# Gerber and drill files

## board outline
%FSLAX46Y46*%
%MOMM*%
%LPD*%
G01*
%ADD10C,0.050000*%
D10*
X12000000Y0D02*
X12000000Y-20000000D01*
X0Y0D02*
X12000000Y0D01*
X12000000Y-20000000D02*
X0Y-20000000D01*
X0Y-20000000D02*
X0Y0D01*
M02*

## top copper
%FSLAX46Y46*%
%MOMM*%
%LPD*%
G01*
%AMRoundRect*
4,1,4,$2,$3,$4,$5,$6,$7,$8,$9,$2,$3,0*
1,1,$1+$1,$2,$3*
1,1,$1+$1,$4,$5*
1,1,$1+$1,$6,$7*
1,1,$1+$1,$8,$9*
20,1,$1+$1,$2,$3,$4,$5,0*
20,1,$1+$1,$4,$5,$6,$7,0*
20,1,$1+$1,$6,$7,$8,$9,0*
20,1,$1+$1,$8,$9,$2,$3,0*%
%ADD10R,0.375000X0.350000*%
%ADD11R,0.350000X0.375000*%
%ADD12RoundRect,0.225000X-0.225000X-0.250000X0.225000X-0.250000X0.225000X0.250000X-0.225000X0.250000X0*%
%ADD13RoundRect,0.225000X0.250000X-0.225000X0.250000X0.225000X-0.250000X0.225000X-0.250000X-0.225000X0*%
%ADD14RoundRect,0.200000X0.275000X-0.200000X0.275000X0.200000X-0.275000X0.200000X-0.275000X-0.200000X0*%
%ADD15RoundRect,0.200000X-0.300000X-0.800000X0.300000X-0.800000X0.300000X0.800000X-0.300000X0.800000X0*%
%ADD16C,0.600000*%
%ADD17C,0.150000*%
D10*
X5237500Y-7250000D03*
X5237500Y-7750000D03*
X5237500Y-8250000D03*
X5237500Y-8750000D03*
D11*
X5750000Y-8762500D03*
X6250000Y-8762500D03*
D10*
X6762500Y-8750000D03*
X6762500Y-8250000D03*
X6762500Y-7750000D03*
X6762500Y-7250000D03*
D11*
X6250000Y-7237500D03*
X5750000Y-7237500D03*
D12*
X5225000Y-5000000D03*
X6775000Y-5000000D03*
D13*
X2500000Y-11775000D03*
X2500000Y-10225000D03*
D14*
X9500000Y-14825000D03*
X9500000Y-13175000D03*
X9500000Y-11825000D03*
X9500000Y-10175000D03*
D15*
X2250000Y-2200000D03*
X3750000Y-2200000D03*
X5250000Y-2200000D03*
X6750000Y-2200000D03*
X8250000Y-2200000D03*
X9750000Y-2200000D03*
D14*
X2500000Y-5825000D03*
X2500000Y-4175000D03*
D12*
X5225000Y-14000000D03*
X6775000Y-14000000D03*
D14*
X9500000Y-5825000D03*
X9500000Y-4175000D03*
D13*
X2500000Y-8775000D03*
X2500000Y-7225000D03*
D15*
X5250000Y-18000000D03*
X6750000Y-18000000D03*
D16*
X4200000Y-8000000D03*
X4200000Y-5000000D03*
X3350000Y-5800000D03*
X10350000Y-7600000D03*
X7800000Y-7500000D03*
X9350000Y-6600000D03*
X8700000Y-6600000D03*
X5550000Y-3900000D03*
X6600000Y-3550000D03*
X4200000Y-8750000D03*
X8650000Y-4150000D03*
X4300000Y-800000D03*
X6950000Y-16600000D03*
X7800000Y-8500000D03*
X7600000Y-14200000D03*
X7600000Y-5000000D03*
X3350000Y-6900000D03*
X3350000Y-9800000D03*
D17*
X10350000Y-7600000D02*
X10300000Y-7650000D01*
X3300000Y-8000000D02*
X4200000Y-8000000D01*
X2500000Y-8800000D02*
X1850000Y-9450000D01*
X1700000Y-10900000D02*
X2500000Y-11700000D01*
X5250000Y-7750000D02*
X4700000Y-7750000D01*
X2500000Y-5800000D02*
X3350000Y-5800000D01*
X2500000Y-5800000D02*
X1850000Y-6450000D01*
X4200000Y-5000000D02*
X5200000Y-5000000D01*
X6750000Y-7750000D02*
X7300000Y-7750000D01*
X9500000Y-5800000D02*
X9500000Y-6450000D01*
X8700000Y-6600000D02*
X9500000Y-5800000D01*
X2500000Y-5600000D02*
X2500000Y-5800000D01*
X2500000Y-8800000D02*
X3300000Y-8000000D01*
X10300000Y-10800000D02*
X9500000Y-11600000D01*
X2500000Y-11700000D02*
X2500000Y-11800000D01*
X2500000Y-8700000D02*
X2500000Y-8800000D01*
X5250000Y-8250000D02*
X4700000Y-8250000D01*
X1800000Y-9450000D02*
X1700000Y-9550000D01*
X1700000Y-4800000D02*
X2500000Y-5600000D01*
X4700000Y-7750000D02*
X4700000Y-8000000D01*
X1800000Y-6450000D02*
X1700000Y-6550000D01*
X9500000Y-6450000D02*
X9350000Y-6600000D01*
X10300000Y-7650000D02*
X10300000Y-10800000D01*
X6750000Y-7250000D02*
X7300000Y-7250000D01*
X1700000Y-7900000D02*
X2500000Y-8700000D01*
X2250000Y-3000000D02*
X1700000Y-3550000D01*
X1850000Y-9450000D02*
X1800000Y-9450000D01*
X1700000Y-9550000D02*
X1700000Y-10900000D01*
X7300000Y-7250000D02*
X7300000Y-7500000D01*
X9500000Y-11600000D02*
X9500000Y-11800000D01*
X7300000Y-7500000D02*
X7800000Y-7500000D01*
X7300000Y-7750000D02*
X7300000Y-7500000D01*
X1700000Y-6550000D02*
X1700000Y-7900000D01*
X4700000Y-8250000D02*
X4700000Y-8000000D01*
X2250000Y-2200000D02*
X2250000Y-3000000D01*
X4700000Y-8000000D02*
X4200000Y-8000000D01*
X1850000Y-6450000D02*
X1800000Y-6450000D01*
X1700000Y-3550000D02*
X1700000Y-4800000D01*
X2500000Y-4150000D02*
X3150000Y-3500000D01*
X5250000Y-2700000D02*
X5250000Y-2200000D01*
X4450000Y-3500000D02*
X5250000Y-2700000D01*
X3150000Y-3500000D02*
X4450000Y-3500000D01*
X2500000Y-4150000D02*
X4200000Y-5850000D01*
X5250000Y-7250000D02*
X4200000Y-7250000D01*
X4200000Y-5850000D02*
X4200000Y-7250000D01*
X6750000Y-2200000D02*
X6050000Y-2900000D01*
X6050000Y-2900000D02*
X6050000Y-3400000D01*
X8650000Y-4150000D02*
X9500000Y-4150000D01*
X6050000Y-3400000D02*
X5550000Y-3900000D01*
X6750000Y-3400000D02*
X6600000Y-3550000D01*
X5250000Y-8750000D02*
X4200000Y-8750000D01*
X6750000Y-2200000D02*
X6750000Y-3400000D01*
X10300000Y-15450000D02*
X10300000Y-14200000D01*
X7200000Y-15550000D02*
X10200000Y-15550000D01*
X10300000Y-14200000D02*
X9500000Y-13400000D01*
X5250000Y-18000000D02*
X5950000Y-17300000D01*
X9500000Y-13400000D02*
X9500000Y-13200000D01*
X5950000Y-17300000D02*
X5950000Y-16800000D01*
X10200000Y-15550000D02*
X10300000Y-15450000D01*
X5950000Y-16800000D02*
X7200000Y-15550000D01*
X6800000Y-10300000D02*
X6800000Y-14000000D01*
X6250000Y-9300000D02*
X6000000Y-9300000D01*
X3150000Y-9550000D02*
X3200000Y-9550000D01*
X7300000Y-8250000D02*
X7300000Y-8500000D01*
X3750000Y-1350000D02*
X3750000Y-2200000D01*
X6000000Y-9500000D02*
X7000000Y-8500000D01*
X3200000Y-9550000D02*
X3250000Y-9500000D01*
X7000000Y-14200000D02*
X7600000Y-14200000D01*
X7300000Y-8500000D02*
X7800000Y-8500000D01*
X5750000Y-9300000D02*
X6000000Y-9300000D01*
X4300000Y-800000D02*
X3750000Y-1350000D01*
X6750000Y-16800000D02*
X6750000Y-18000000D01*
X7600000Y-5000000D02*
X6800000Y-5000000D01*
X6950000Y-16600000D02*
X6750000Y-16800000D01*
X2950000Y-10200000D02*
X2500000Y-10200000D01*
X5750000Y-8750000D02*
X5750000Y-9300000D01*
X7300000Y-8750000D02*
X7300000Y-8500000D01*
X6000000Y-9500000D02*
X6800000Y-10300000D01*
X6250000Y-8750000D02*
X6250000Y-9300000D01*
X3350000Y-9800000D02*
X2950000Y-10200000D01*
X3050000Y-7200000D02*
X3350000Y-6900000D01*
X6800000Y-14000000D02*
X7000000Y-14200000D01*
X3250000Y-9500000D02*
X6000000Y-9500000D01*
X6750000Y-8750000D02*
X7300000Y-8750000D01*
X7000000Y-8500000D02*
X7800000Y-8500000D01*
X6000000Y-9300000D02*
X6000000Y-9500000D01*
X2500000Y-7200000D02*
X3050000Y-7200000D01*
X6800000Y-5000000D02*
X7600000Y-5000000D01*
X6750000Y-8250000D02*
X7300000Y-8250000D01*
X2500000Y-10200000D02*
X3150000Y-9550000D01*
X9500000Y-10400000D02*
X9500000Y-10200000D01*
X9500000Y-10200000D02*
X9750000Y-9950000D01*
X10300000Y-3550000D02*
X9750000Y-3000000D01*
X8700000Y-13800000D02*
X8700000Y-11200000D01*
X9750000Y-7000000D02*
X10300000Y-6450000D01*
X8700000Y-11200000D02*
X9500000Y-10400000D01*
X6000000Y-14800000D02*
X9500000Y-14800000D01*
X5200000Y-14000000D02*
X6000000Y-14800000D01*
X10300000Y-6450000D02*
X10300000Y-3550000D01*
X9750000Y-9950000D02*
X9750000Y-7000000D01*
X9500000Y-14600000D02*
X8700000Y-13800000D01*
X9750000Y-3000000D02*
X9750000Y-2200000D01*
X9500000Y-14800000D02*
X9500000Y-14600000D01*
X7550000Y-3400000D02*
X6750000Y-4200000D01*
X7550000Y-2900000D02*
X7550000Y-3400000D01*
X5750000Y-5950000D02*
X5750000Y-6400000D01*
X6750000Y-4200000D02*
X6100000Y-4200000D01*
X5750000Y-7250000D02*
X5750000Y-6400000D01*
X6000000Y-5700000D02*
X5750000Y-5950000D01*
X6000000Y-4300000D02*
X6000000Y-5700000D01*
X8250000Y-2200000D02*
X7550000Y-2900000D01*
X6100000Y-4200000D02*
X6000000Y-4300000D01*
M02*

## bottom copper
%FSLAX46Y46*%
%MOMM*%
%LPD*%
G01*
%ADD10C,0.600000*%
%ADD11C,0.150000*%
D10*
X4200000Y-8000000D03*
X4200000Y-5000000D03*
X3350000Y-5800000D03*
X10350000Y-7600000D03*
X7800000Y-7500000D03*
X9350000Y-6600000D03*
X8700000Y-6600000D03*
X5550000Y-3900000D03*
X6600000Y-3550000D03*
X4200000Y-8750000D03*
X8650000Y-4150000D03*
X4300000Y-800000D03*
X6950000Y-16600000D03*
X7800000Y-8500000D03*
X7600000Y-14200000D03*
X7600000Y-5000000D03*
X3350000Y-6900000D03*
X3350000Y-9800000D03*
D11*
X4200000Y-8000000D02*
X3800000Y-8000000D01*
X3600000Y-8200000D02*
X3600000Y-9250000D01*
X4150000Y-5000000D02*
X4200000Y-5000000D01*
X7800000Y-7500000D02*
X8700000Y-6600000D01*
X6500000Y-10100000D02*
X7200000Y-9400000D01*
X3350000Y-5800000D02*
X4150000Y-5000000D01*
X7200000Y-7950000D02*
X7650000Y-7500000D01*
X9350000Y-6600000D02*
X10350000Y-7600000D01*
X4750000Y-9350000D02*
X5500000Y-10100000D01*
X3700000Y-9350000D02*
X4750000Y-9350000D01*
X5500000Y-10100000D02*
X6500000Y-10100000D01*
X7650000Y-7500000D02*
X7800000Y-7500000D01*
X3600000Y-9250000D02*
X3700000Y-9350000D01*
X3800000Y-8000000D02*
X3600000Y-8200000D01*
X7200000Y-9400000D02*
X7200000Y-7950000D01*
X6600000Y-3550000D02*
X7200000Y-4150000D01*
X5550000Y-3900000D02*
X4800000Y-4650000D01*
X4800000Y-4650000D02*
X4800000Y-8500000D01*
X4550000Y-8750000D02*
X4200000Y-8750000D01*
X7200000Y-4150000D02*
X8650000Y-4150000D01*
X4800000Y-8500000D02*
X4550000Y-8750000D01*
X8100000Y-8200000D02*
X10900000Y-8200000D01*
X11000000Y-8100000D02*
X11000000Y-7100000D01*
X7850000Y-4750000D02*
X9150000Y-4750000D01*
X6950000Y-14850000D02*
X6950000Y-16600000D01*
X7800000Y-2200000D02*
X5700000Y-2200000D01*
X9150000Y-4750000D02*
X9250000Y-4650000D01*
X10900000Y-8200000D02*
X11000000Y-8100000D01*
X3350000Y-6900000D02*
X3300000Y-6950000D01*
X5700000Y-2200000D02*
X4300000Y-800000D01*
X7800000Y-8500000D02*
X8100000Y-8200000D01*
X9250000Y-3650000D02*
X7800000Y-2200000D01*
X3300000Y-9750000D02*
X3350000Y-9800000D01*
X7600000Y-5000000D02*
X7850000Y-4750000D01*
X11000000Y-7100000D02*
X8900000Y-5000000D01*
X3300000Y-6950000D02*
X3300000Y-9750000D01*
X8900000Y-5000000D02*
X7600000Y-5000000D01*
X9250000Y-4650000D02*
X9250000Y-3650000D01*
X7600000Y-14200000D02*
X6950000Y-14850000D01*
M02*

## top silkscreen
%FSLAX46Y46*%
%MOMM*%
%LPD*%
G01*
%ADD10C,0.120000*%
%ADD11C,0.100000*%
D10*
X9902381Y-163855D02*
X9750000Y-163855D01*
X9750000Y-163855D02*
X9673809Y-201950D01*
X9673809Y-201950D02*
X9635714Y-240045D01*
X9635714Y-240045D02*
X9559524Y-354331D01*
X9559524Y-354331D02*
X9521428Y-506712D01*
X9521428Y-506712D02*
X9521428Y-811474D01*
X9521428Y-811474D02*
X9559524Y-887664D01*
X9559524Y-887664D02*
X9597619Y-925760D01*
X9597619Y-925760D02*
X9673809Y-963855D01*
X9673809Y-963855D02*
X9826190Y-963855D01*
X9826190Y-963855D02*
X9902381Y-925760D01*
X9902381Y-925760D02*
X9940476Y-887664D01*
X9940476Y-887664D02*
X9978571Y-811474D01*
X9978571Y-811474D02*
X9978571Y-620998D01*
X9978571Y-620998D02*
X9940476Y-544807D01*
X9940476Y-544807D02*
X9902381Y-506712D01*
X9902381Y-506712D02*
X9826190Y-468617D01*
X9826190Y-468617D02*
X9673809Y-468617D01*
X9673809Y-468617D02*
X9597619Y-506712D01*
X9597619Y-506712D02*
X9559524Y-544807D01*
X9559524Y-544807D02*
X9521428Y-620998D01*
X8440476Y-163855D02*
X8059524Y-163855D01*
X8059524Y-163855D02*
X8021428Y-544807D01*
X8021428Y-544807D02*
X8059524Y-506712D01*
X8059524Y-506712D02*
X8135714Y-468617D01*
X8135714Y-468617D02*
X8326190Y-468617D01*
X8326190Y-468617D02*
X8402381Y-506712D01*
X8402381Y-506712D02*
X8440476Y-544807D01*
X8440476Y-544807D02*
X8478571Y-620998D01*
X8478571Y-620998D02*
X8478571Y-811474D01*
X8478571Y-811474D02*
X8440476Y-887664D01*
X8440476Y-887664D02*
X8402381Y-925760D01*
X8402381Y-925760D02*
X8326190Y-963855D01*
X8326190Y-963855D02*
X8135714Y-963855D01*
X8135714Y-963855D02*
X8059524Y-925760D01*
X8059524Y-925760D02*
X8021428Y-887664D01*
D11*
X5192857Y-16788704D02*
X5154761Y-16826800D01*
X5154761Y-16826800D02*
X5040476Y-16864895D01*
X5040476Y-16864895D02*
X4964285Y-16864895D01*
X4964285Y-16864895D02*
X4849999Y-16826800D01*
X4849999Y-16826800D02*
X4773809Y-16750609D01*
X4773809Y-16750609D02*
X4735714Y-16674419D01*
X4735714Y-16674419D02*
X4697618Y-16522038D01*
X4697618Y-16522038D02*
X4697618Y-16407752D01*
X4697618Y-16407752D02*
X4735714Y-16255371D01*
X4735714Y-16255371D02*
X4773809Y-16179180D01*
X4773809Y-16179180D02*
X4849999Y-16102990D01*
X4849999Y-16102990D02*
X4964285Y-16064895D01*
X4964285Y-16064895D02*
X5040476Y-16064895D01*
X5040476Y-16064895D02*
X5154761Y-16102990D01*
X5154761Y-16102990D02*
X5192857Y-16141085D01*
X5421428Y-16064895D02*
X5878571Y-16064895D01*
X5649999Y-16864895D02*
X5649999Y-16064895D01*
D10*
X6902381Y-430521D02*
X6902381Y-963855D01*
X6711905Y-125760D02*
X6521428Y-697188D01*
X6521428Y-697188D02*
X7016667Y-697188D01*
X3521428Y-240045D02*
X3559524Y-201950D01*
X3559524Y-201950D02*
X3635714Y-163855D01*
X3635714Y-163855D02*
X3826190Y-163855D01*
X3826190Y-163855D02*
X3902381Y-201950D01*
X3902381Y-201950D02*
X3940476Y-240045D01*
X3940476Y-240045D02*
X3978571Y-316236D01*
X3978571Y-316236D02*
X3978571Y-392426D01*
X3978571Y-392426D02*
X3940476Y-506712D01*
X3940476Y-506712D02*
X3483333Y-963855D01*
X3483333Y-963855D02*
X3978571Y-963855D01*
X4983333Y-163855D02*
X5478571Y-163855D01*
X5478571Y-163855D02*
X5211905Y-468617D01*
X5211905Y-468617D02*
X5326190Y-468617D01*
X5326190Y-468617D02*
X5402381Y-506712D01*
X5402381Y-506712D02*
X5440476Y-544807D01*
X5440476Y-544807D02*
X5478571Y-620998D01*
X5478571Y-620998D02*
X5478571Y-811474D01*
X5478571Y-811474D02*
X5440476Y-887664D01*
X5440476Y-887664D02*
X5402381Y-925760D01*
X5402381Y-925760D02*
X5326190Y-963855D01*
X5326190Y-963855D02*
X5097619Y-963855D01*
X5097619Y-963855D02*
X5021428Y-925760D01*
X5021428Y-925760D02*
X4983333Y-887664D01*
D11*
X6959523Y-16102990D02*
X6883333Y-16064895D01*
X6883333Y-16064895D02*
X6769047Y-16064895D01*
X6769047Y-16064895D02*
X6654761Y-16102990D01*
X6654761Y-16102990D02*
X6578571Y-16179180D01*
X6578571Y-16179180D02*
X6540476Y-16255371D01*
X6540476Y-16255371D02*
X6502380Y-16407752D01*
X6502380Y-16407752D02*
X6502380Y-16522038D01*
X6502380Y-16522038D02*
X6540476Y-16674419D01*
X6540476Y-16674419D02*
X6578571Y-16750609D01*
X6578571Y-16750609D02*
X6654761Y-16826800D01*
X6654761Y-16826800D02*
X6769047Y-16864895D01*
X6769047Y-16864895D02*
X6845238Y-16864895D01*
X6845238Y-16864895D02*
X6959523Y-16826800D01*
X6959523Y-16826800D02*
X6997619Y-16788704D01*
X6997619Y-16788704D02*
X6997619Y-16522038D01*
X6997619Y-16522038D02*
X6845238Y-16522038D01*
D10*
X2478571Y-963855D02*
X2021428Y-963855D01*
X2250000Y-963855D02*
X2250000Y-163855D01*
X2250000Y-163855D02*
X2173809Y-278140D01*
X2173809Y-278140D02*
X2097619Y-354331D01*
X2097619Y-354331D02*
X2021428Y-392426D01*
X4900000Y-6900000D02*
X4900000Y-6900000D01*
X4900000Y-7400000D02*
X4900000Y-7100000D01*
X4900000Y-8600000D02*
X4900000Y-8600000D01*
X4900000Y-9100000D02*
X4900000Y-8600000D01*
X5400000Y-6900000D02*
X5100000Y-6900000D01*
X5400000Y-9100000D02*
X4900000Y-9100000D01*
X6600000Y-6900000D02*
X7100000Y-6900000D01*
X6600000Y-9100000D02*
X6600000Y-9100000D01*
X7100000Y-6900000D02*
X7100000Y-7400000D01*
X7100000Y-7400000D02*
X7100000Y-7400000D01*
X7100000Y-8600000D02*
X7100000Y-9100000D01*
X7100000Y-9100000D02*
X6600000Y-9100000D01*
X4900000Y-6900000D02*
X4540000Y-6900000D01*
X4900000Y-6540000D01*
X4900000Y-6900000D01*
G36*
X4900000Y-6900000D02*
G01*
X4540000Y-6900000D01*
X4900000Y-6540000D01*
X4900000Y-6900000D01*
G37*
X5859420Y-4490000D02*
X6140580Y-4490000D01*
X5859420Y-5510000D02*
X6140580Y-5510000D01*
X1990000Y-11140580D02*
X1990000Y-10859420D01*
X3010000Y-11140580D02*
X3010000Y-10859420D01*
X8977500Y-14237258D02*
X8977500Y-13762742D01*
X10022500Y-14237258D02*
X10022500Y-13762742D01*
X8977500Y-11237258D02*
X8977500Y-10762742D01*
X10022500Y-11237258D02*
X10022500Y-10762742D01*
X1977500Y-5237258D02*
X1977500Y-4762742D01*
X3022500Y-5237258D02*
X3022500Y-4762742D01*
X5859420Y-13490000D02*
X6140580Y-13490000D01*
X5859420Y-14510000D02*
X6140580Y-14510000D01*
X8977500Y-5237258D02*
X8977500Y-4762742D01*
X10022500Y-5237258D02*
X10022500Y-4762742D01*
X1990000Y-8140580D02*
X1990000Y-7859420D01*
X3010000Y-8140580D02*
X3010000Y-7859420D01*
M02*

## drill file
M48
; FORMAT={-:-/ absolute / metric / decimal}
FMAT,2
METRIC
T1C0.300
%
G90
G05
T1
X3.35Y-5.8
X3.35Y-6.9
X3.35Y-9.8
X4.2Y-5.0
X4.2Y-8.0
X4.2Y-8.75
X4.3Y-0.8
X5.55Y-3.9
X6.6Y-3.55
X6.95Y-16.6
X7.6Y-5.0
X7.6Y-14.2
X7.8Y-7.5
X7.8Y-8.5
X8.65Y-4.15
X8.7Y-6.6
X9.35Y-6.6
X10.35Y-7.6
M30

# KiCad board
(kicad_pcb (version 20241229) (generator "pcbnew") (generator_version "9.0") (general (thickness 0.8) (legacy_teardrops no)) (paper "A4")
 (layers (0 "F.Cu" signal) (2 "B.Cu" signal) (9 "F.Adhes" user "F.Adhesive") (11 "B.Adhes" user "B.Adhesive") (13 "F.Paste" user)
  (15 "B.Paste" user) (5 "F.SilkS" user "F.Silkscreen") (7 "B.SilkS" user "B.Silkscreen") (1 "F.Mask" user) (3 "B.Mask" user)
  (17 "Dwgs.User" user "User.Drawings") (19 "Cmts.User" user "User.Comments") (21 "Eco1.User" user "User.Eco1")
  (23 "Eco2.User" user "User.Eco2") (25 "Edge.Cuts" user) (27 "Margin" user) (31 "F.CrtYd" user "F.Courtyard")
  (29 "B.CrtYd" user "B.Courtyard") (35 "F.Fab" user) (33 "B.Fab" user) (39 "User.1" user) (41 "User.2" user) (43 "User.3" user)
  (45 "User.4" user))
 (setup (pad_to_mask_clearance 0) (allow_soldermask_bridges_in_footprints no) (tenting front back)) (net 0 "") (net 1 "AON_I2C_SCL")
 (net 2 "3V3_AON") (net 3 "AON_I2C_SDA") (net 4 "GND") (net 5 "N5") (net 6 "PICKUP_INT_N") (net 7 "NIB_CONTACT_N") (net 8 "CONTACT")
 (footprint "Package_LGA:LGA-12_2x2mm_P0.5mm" (layer "F.Cu") (at 6 8)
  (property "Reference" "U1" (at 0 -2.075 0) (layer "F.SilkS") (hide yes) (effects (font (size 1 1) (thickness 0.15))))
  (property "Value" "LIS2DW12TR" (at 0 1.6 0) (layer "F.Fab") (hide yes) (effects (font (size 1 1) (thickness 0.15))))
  (fp_line (start -1.1 -1.1) (end -1.1 -1.1) (stroke (width 0.12) (type solid)) (layer "F.SilkS"))
  (fp_line (start -1.1 -0.6) (end -1.1 -0.9) (stroke (width 0.12) (type solid)) (layer "F.SilkS"))
  (fp_line (start -1.1 0.6) (end -1.1 0.6) (stroke (width 0.12) (type solid)) (layer "F.SilkS"))
  (fp_line (start -1.1 1.1) (end -1.1 0.6) (stroke (width 0.12) (type solid)) (layer "F.SilkS"))
  (fp_line (start -0.6 -1.1) (end -0.9 -1.1) (stroke (width 0.12) (type solid)) (layer "F.SilkS"))
  (fp_line (start -0.6 1.1) (end -1.1 1.1) (stroke (width 0.12) (type solid)) (layer "F.SilkS"))
  (fp_line (start 0.6 -1.1) (end 1.1 -1.1) (stroke (width 0.12) (type solid)) (layer "F.SilkS"))
  (fp_line (start 0.6 1.1) (end 0.6 1.1) (stroke (width 0.12) (type solid)) (layer "F.SilkS"))
  (fp_line (start 1.1 -1.1) (end 1.1 -0.6) (stroke (width 0.12) (type solid)) (layer "F.SilkS"))
  (fp_line (start 1.1 -0.6) (end 1.1 -0.6) (stroke (width 0.12) (type solid)) (layer "F.SilkS"))
  (fp_line (start 1.1 0.6) (end 1.1 1.1) (stroke (width 0.12) (type solid)) (layer "F.SilkS"))
  (fp_line (start 1.1 1.1) (end 0.6 1.1) (stroke (width 0.12) (type solid)) (layer "F.SilkS"))
  (fp_poly
   (pts (xy -1.1 -1.1) (xy -1.46 -1.1) (xy -1.1 -1.46) (xy -1.1 -1.1)) (stroke (width 0.12) (type solid)) (fill yes) (layer "F.SilkS"))
  (pad "1" smd rect (at -0.7625 -0.75) (size 0.375 0.35) (layers "F.Cu" "F.Mask" "F.Paste") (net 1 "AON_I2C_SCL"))
  (pad "2" smd rect (at -0.7625 -0.25) (size 0.375 0.35) (layers "F.Cu" "F.Mask" "F.Paste") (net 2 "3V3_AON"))
  (pad "3" smd rect (at -0.7625 0.25) (size 0.375 0.35) (layers "F.Cu" "F.Mask" "F.Paste") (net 2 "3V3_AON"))
  (pad "4" smd rect (at -0.7625 0.75) (size 0.375 0.35) (layers "F.Cu" "F.Mask" "F.Paste") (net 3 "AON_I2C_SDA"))
  (pad "5" smd rect (at -0.25 0.7625 90) (size 0.375 0.35) (layers "F.Cu" "F.Mask" "F.Paste") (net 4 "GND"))
  (pad "6" smd rect (at 0.25 0.7625 90) (size 0.375 0.35) (layers "F.Cu" "F.Mask" "F.Paste") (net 4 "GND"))
  (pad "7" smd rect (at 0.7625 0.75) (size 0.375 0.35) (layers "F.Cu" "F.Mask" "F.Paste") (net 4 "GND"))
  (pad "8" smd rect (at 0.7625 0.25) (size 0.375 0.35) (layers "F.Cu" "F.Mask" "F.Paste") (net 4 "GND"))
  (pad "9" smd rect (at 0.7625 -0.25) (size 0.375 0.35) (layers "F.Cu" "F.Mask" "F.Paste") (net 2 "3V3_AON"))
  (pad "10" smd rect (at 0.7625 -0.75) (size 0.375 0.35) (layers "F.Cu" "F.Mask" "F.Paste") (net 2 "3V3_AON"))
  (pad "11" smd rect (at 0.25 -0.7625 90) (size 0.375 0.35) (layers "F.Cu" "F.Mask" "F.Paste") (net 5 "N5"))
  (pad "12" smd rect (at -0.25 -0.7625 90) (size 0.375 0.35) (layers "F.Cu" "F.Mask" "F.Paste") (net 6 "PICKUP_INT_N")))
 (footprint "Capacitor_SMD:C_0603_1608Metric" (layer "F.Cu") (at 6 5)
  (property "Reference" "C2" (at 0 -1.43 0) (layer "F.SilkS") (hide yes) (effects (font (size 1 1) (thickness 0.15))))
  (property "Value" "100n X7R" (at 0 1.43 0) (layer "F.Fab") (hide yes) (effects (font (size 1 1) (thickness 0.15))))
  (fp_line (start -0.14058 -0.51) (end 0.14058 -0.51) (stroke (width 0.12) (type solid)) (layer "F.SilkS"))
  (fp_line (start -0.14058 0.51) (end 0.14058 0.51) (stroke (width 0.12) (type solid)) (layer "F.SilkS"))
  (pad "1" smd roundrect (at -0.775 0) (size 0.9 0.95) (layers "F.Cu" "F.Mask" "F.Paste") (roundrect_rratio 0.25) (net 2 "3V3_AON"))
  (pad "2" smd roundrect (at 0.775 0) (size 0.9 0.95) (layers "F.Cu" "F.Mask" "F.Paste") (roundrect_rratio 0.25) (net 4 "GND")))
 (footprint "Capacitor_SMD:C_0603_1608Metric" (layer "F.Cu") (at 2.5 11 90)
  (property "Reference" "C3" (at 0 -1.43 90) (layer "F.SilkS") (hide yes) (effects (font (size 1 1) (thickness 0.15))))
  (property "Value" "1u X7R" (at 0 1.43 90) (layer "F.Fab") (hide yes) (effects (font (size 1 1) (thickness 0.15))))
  (fp_line (start -0.14058 -0.51) (end 0.14058 -0.51) (stroke (width 0.12) (type solid)) (layer "F.SilkS"))
  (fp_line (start -0.14058 0.51) (end 0.14058 0.51) (stroke (width 0.12) (type solid)) (layer "F.SilkS"))
  (pad "1" smd roundrect (at -0.775 0 90) (size 0.9 0.95) (layers "F.Cu" "F.Mask" "F.Paste") (roundrect_rratio 0.25) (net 2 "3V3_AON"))
  (pad "2" smd roundrect (at 0.775 0 90) (size 0.9 0.95) (layers "F.Cu" "F.Mask" "F.Paste") (roundrect_rratio 0.25) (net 4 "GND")))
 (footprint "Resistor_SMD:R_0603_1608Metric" (layer "F.Cu") (at 9.5 14 90)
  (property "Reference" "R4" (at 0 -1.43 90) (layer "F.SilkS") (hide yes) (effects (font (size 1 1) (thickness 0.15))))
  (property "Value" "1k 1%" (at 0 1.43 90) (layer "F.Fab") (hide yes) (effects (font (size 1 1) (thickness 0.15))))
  (fp_line (start -0.237258 -0.5225) (end 0.237258 -0.5225) (stroke (width 0.12) (type solid)) (layer "F.SilkS"))
  (fp_line (start -0.237258 0.5225) (end 0.237258 0.5225) (stroke (width 0.12) (type solid)) (layer "F.SilkS"))
  (pad "1" smd roundrect (at -0.825 0 90) (size 0.8 0.95) (layers "F.Cu" "F.Mask" "F.Paste") (roundrect_rratio 0.25) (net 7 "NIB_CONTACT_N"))
  (pad "2" smd roundrect (at 0.825 0 90) (size 0.8 0.95) (layers "F.Cu" "F.Mask" "F.Paste") (roundrect_rratio 0.25) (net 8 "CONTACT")))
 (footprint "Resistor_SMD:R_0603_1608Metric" (layer "F.Cu") (at 9.5 11 90)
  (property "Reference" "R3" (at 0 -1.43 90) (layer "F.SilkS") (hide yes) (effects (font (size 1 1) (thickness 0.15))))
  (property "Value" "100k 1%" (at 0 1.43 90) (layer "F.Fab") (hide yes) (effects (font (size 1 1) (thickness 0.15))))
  (fp_line (start -0.237258 -0.5225) (end 0.237258 -0.5225) (stroke (width 0.12) (type solid)) (layer "F.SilkS"))
  (fp_line (start -0.237258 0.5225) (end 0.237258 0.5225) (stroke (width 0.12) (type solid)) (layer "F.SilkS"))
  (pad "1" smd roundrect (at -0.825 0 90) (size 0.8 0.95) (layers "F.Cu" "F.Mask" "F.Paste") (roundrect_rratio 0.25) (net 2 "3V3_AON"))
  (pad "2" smd roundrect (at 0.825 0 90) (size 0.8 0.95) (layers "F.Cu" "F.Mask" "F.Paste") (roundrect_rratio 0.25) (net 7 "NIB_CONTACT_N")))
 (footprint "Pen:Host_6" (layer "F.Cu") (at 2.25 2.2)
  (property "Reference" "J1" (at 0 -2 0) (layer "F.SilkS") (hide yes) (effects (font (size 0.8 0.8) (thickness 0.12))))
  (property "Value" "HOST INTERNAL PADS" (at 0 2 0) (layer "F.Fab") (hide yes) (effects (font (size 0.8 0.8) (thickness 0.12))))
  (pad "1" smd roundrect (at 0 0) (size 1 2) (layers "F.Cu" "F.Mask") (roundrect_rratio 0.2) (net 2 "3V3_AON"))
  (pad "2" smd roundrect (at 1.5 0) (size 1 2) (layers "F.Cu" "F.Mask") (roundrect_rratio 0.2) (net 4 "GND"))
  (pad "3" smd roundrect (at 3 0) (size 1 2) (layers "F.Cu" "F.Mask") (roundrect_rratio 0.2) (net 1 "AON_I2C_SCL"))
  (pad "4" smd roundrect (at 4.5 0) (size 1 2) (layers "F.Cu" "F.Mask") (roundrect_rratio 0.2) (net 3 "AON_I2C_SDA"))
  (pad "5" smd roundrect (at 6 0) (size 1 2) (layers "F.Cu" "F.Mask") (roundrect_rratio 0.2) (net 6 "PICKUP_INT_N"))
  (pad "6" smd roundrect (at 7.5 0) (size 1 2) (layers "F.Cu" "F.Mask") (roundrect_rratio 0.2) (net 7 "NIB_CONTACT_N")))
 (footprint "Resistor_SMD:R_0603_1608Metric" (layer "F.Cu") (at 2.5 5 90)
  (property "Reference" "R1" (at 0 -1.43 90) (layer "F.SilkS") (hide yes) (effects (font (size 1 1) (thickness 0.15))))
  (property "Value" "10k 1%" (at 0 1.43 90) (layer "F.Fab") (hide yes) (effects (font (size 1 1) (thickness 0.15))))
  (fp_line (start -0.237258 -0.5225) (end 0.237258 -0.5225) (stroke (width 0.12) (type solid)) (layer "F.SilkS"))
  (fp_line (start -0.237258 0.5225) (end 0.237258 0.5225) (stroke (width 0.12) (type solid)) (layer "F.SilkS"))
  (pad "1" smd roundrect (at -0.825 0 90) (size 0.8 0.95) (layers "F.Cu" "F.Mask" "F.Paste") (roundrect_rratio 0.25) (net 2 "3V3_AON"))
  (pad "2" smd roundrect (at 0.825 0 90) (size 0.8 0.95) (layers "F.Cu" "F.Mask" "F.Paste") (roundrect_rratio 0.25) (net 1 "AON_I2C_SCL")))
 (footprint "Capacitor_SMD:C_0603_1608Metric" (layer "F.Cu") (at 6 14)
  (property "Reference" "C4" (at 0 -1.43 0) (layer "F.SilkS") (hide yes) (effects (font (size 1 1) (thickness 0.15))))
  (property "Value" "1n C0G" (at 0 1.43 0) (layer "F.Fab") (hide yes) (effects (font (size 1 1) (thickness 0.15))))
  (fp_line (start -0.14058 -0.51) (end 0.14058 -0.51) (stroke (width 0.12) (type solid)) (layer "F.SilkS"))
  (fp_line (start -0.14058 0.51) (end 0.14058 0.51) (stroke (width 0.12) (type solid)) (layer "F.SilkS"))
  (pad "1" smd roundrect (at -0.775 0) (size 0.9 0.95) (layers "F.Cu" "F.Mask" "F.Paste") (roundrect_rratio 0.25) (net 7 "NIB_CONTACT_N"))
  (pad "2" smd roundrect (at 0.775 0) (size 0.9 0.95) (layers "F.Cu" "F.Mask" "F.Paste") (roundrect_rratio 0.25) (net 4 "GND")))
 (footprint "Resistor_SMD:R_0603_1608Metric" (layer "F.Cu") (at 9.5 5 90)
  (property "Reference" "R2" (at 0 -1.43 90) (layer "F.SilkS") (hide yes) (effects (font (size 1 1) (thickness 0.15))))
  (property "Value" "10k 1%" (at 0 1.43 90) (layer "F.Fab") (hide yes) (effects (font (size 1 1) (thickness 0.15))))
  (fp_line (start -0.237258 -0.5225) (end 0.237258 -0.5225) (stroke (width 0.12) (type solid)) (layer "F.SilkS"))
  (fp_line (start -0.237258 0.5225) (end 0.237258 0.5225) (stroke (width 0.12) (type solid)) (layer "F.SilkS"))
  (pad "1" smd roundrect (at -0.825 0 90) (size 0.8 0.95) (layers "F.Cu" "F.Mask" "F.Paste") (roundrect_rratio 0.25) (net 2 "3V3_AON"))
  (pad "2" smd roundrect (at 0.825 0 90) (size 0.8 0.95) (layers "F.Cu" "F.Mask" "F.Paste") (roundrect_rratio 0.25) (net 3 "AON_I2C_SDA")))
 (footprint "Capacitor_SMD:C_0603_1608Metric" (layer "F.Cu") (at 2.5 8 90)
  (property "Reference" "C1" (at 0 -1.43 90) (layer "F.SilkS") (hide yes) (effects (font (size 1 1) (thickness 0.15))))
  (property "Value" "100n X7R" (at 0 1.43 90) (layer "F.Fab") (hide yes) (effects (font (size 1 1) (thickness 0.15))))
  (fp_line (start -0.14058 -0.51) (end 0.14058 -0.51) (stroke (width 0.12) (type solid)) (layer "F.SilkS"))
  (fp_line (start -0.14058 0.51) (end 0.14058 0.51) (stroke (width 0.12) (type solid)) (layer "F.SilkS"))
  (pad "1" smd roundrect (at -0.775 0 90) (size 0.9 0.95) (layers "F.Cu" "F.Mask" "F.Paste") (roundrect_rratio 0.25) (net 2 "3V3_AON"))
  (pad "2" smd roundrect (at 0.775 0 90) (size 0.9 0.95) (layers "F.Cu" "F.Mask" "F.Paste") (roundrect_rratio 0.25) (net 4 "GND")))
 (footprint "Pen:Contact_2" (layer "F.Cu") (at 5.25 18)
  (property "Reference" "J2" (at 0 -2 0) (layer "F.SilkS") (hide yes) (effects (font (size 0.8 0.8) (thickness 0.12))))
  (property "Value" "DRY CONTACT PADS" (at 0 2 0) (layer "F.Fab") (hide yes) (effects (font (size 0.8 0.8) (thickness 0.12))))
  (pad "1" smd roundrect (at 0 0) (size 1 2) (layers "F.Cu" "F.Mask") (roundrect_rratio 0.2) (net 8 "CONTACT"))
  (pad "2" smd roundrect (at 1.5 0) (size 1 2) (layers "F.Cu" "F.Mask") (roundrect_rratio 0.2) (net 4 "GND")))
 (gr_line (start 12 0) (end 12 20) (stroke (width 0.05) (type default)) (layer "Edge.Cuts"))
 (gr_line (start 0 0) (end 12 0) (stroke (width 0.05) (type default)) (layer "Edge.Cuts"))
 (gr_line (start 12 20) (end 0 20) (stroke (width 0.05) (type default)) (layer "Edge.Cuts"))
 (gr_line (start 0 20) (end 0 0) (stroke (width 0.05) (type default)) (layer "Edge.Cuts"))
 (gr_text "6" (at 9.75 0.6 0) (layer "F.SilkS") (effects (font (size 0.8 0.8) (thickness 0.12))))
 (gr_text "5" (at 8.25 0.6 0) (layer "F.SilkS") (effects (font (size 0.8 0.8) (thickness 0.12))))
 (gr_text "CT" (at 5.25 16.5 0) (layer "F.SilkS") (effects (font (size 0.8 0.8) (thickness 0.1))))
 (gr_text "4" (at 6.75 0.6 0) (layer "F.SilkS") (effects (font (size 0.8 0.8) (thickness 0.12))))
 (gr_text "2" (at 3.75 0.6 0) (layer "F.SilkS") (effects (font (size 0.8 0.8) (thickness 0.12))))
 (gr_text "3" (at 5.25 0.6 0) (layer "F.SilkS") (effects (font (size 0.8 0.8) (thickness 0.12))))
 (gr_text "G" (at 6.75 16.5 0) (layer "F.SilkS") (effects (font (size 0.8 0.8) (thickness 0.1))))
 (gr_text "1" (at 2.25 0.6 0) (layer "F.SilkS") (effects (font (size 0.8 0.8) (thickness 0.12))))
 (segment (start 10.35 7.6) (end 10.3 7.65) (width 0.15) (layer "F.Cu") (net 2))
 (segment (start 3.3 8) (end 4.2 8) (width 0.15) (layer "F.Cu") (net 2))
 (segment (start 2.5 8.8) (end 1.85 9.45) (width 0.15) (layer "F.Cu") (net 2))
 (segment (start 1.7 10.9) (end 2.5 11.7) (width 0.15) (layer "F.Cu") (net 2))
 (segment (start 5.25 7.75) (end 4.7 7.75) (width 0.15) (layer "F.Cu") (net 2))
 (segment (start 2.5 5.8) (end 3.35 5.8) (width 0.15) (layer "F.Cu") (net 2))
 (segment (start 2.5 5.8) (end 1.85 6.45) (width 0.15) (layer "F.Cu") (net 2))
 (segment (start 4.2 5) (end 5.2 5) (width 0.15) (layer "F.Cu") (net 2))
 (segment (start 6.75 7.75) (end 7.3 7.75) (width 0.15) (layer "F.Cu") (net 2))
 (segment (start 9.5 5.8) (end 9.5 6.45) (width 0.15) (layer "F.Cu") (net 2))
 (segment (start 8.7 6.6) (end 9.5 5.8) (width 0.15) (layer "F.Cu") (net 2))
 (segment (start 2.5 5.6) (end 2.5 5.8) (width 0.15) (layer "F.Cu") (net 2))
 (segment (start 2.5 8.8) (end 3.3 8) (width 0.15) (layer "F.Cu") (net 2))
 (segment (start 10.3 10.8) (end 9.5 11.6) (width 0.15) (layer "F.Cu") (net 2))
 (segment (start 2.5 11.7) (end 2.5 11.8) (width 0.15) (layer "F.Cu") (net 2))
 (segment (start 2.5 8.7) (end 2.5 8.8) (width 0.15) (layer "F.Cu") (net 2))
 (segment (start 5.25 8.25) (end 4.7 8.25) (width 0.15) (layer "F.Cu") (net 2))
 (segment (start 1.8 9.45) (end 1.7 9.55) (width 0.15) (layer "F.Cu") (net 2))
 (segment (start 1.7 4.8) (end 2.5 5.6) (width 0.15) (layer "F.Cu") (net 2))
 (segment (start 4.7 7.75) (end 4.7 8) (width 0.15) (layer "F.Cu") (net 2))
 (segment (start 1.8 6.45) (end 1.7 6.55) (width 0.15) (layer "F.Cu") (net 2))
 (segment (start 9.5 6.45) (end 9.35 6.6) (width 0.15) (layer "F.Cu") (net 2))
 (segment (start 10.3 7.65) (end 10.3 10.8) (width 0.15) (layer "F.Cu") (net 2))
 (segment (start 6.75 7.25) (end 7.3 7.25) (width 0.15) (layer "F.Cu") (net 2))
 (segment (start 1.7 7.9) (end 2.5 8.7) (width 0.15) (layer "F.Cu") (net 2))
 (segment (start 2.25 3) (end 1.7 3.55) (width 0.15) (layer "F.Cu") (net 2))
 (segment (start 1.85 9.45) (end 1.8 9.45) (width 0.15) (layer "F.Cu") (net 2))
 (segment (start 1.7 9.55) (end 1.7 10.9) (width 0.15) (layer "F.Cu") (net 2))
 (segment (start 7.3 7.25) (end 7.3 7.5) (width 0.15) (layer "F.Cu") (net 2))
 (segment (start 9.5 11.6) (end 9.5 11.8) (width 0.15) (layer "F.Cu") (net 2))
 (segment (start 7.3 7.5) (end 7.8 7.5) (width 0.15) (layer "F.Cu") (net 2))
 (segment (start 7.3 7.75) (end 7.3 7.5) (width 0.15) (layer "F.Cu") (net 2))
 (segment (start 1.7 6.55) (end 1.7 7.9) (width 0.15) (layer "F.Cu") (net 2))
 (segment (start 4.7 8.25) (end 4.7 8) (width 0.15) (layer "F.Cu") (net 2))
 (segment (start 2.25 2.2) (end 2.25 3) (width 0.15) (layer "F.Cu") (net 2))
 (segment (start 4.7 8) (end 4.2 8) (width 0.15) (layer "F.Cu") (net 2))
 (segment (start 1.85 6.45) (end 1.8 6.45) (width 0.15) (layer "F.Cu") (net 2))
 (segment (start 1.7 3.55) (end 1.7 4.8) (width 0.15) (layer "F.Cu") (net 2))
 (via (at 4.2 8) (size 0.6) (drill 0.3) (layers "F.Cu" "B.Cu") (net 2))
 (via (at 4.2 5) (size 0.6) (drill 0.3) (layers "F.Cu" "B.Cu") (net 2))
 (via (at 3.35 5.8) (size 0.6) (drill 0.3) (layers "F.Cu" "B.Cu") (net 2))
 (via (at 10.35 7.6) (size 0.6) (drill 0.3) (layers "F.Cu" "B.Cu") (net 2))
 (via (at 7.8 7.5) (size 0.6) (drill 0.3) (layers "F.Cu" "B.Cu") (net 2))
 (via (at 9.35 6.6) (size 0.6) (drill 0.3) (layers "F.Cu" "B.Cu") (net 2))
 (via (at 8.7 6.6) (size 0.6) (drill 0.3) (layers "F.Cu" "B.Cu") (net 2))
 (segment (start 4.2 8) (end 3.8 8) (width 0.15) (layer "B.Cu") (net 2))
 (segment (start 3.6 8.2) (end 3.6 9.25) (width 0.15) (layer "B.Cu") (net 2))
 (segment (start 4.15 5) (end 4.2 5) (width 0.15) (layer "B.Cu") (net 2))
 (segment (start 7.8 7.5) (end 8.7 6.6) (width 0.15) (layer "B.Cu") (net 2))
 (segment (start 6.5 10.1) (end 7.2 9.4) (width 0.15) (layer "B.Cu") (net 2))
 (segment (start 3.35 5.8) (end 4.15 5) (width 0.15) (layer "B.Cu") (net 2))
 (segment (start 7.2 7.95) (end 7.65 7.5) (width 0.15) (layer "B.Cu") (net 2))
 (segment (start 9.35 6.6) (end 10.35 7.6) (width 0.15) (layer "B.Cu") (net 2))
 (segment (start 4.75 9.35) (end 5.5 10.1) (width 0.15) (layer "B.Cu") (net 2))
 (segment (start 3.7 9.35) (end 4.75 9.35) (width 0.15) (layer "B.Cu") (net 2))
 (segment (start 5.5 10.1) (end 6.5 10.1) (width 0.15) (layer "B.Cu") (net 2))
 (segment (start 7.65 7.5) (end 7.8 7.5) (width 0.15) (layer "B.Cu") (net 2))
 (segment (start 3.6 9.25) (end 3.7 9.35) (width 0.15) (layer "B.Cu") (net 2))
 (segment (start 3.8 8) (end 3.6 8.2) (width 0.15) (layer "B.Cu") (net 2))
 (segment (start 7.2 9.4) (end 7.2 7.95) (width 0.15) (layer "B.Cu") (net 2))
 (segment (start 2.5 4.15) (end 3.15 3.5) (width 0.15) (layer "F.Cu") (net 1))
 (segment (start 5.25 2.7) (end 5.25 2.2) (width 0.15) (layer "F.Cu") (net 1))
 (segment (start 4.45 3.5) (end 5.25 2.7) (width 0.15) (layer "F.Cu") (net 1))
 (segment (start 3.15 3.5) (end 4.45 3.5) (width 0.15) (layer "F.Cu") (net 1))
 (segment (start 2.5 4.15) (end 4.2 5.85) (width 0.15) (layer "F.Cu") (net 1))
 (segment (start 5.25 7.25) (end 4.2 7.25) (width 0.15) (layer "F.Cu") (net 1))
 (segment (start 4.2 5.85) (end 4.2 7.25) (width 0.15) (layer "F.Cu") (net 1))
 (segment (start 6.75 2.2) (end 6.05 2.9) (width 0.15) (layer "F.Cu") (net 3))
 (segment (start 6.05 2.9) (end 6.05 3.4) (width 0.15) (layer "F.Cu") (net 3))
 (segment (start 8.65 4.15) (end 9.5 4.15) (width 0.15) (layer "F.Cu") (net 3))
 (segment (start 6.05 3.4) (end 5.55 3.9) (width 0.15) (layer "F.Cu") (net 3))
 (segment (start 6.75 3.4) (end 6.6 3.55) (width 0.15) (layer "F.Cu") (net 3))
 (segment (start 5.25 8.75) (end 4.2 8.75) (width 0.15) (layer "F.Cu") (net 3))
 (segment (start 6.75 2.2) (end 6.75 3.4) (width 0.15) (layer "F.Cu") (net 3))
 (via (at 5.55 3.9) (size 0.6) (drill 0.3) (layers "F.Cu" "B.Cu") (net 3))
 (via (at 6.6 3.55) (size 0.6) (drill 0.3) (layers "F.Cu" "B.Cu") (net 3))
 (via (at 4.2 8.75) (size 0.6) (drill 0.3) (layers "F.Cu" "B.Cu") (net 3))
 (via (at 8.65 4.15) (size 0.6) (drill 0.3) (layers "F.Cu" "B.Cu") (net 3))
 (segment (start 6.6 3.55) (end 7.2 4.15) (width 0.15) (layer "B.Cu") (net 3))
 (segment (start 5.55 3.9) (end 4.8 4.65) (width 0.15) (layer "B.Cu") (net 3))
 (segment (start 4.8 4.65) (end 4.8 8.5) (width 0.15) (layer "B.Cu") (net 3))
 (segment (start 4.55 8.75) (end 4.2 8.75) (width 0.15) (layer "B.Cu") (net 3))
 (segment (start 7.2 4.15) (end 8.65 4.15) (width 0.15) (layer "B.Cu") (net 3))
 (segment (start 4.8 8.5) (end 4.55 8.75) (width 0.15) (layer "B.Cu") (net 3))
 (segment (start 10.3 15.45) (end 10.3 14.2) (width 0.15) (layer "F.Cu") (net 8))
 (segment (start 7.2 15.55) (end 10.2 15.55) (width 0.15) (layer "F.Cu") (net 8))
 (segment (start 10.3 14.2) (end 9.5 13.4) (width 0.15) (layer "F.Cu") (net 8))
 (segment (start 5.25 18) (end 5.95 17.3) (width 0.15) (layer "F.Cu") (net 8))
 (segment (start 9.5 13.4) (end 9.5 13.2) (width 0.15) (layer "F.Cu") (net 8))
 (segment (start 5.95 17.3) (end 5.95 16.8) (width 0.15) (layer "F.Cu") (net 8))
 (segment (start 10.2 15.55) (end 10.3 15.45) (width 0.15) (layer "F.Cu") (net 8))
 (segment (start 5.95 16.8) (end 7.2 15.55) (width 0.15) (layer "F.Cu") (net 8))
 (segment (start 6.8 10.3) (end 6.8 14) (width 0.15) (layer "F.Cu") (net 4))
 (segment (start 6.25 9.3) (end 6 9.3) (width 0.15) (layer "F.Cu") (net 4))
 (segment (start 3.15 9.55) (end 3.2 9.55) (width 0.15) (layer "F.Cu") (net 4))
 (segment (start 7.3 8.25) (end 7.3 8.5) (width 0.15) (layer "F.Cu") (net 4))
 (segment (start 3.75 1.35) (end 3.75 2.2) (width 0.15) (layer "F.Cu") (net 4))
 (segment (start 6 9.5) (end 7 8.5) (width 0.15) (layer "F.Cu") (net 4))
 (segment (start 3.2 9.55) (end 3.25 9.5) (width 0.15) (layer "F.Cu") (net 4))
 (segment (start 7 14.2) (end 7.6 14.2) (width 0.15) (layer "F.Cu") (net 4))
 (segment (start 7.3 8.5) (end 7.8 8.5) (width 0.15) (layer "F.Cu") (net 4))
 (segment (start 5.75 9.3) (end 6 9.3) (width 0.15) (layer "F.Cu") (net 4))
 (segment (start 4.3 0.8) (end 3.75 1.35) (width 0.15) (layer "F.Cu") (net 4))
 (segment (start 6.75 16.8) (end 6.75 18) (width 0.15) (layer "F.Cu") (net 4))
 (segment (start 7.6 5) (end 6.8 5) (width 0.15) (layer "F.Cu") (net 4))
 (segment (start 6.95 16.6) (end 6.75 16.8) (width 0.15) (layer "F.Cu") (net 4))
 (segment (start 2.95 10.2) (end 2.5 10.2) (width 0.15) (layer "F.Cu") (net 4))
 (segment (start 5.75 8.75) (end 5.75 9.3) (width 0.15) (layer "F.Cu") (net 4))
 (segment (start 7.3 8.75) (end 7.3 8.5) (width 0.15) (layer "F.Cu") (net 4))
 (segment (start 6 9.5) (end 6.8 10.3) (width 0.15) (layer "F.Cu") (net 4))
 (segment (start 6.25 8.75) (end 6.25 9.3) (width 0.15) (layer "F.Cu") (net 4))
 (segment (start 3.35 9.8) (end 2.95 10.2) (width 0.15) (layer "F.Cu") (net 4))
 (segment (start 3.05 7.2) (end 3.35 6.9) (width 0.15) (layer "F.Cu") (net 4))
 (segment (start 6.8 14) (end 7 14.2) (width 0.15) (layer "F.Cu") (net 4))
 (segment (start 3.25 9.5) (end 6 9.5) (width 0.15) (layer "F.Cu") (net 4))
 (segment (start 6.75 8.75) (end 7.3 8.75) (width 0.15) (layer "F.Cu") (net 4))
 (segment (start 7 8.5) (end 7.8 8.5) (width 0.15) (layer "F.Cu") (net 4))
 (segment (start 6 9.3) (end 6 9.5) (width 0.15) (layer "F.Cu") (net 4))
 (segment (start 2.5 7.2) (end 3.05 7.2) (width 0.15) (layer "F.Cu") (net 4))
 (segment (start 6.8 5) (end 7.6 5) (width 0.15) (layer "F.Cu") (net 4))
 (segment (start 6.75 8.25) (end 7.3 8.25) (width 0.15) (layer "F.Cu") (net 4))
 (segment (start 2.5 10.2) (end 3.15 9.55) (width 0.15) (layer "F.Cu") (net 4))
 (via (at 4.3 0.8) (size 0.6) (drill 0.3) (layers "F.Cu" "B.Cu") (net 4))
 (via (at 6.95 16.6) (size 0.6) (drill 0.3) (layers "F.Cu" "B.Cu") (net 4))
 (via (at 7.8 8.5) (size 0.6) (drill 0.3) (layers "F.Cu" "B.Cu") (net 4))
 (via (at 7.6 14.2) (size 0.6) (drill 0.3) (layers "F.Cu" "B.Cu") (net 4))
 (via (at 7.6 5) (size 0.6) (drill 0.3) (layers "F.Cu" "B.Cu") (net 4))
 (via (at 3.35 6.9) (size 0.6) (drill 0.3) (layers "F.Cu" "B.Cu") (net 4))
 (via (at 3.35 9.8) (size 0.6) (drill 0.3) (layers "F.Cu" "B.Cu") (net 4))
 (segment (start 8.1 8.2) (end 10.9 8.2) (width 0.15) (layer "B.Cu") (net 4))
 (segment (start 11 8.1) (end 11 7.1) (width 0.15) (layer "B.Cu") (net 4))
 (segment (start 7.85 4.75) (end 9.15 4.75) (width 0.15) (layer "B.Cu") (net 4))
 (segment (start 6.95 14.85) (end 6.95 16.6) (width 0.15) (layer "B.Cu") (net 4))
 (segment (start 7.8 2.2) (end 5.7 2.2) (width 0.15) (layer "B.Cu") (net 4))
 (segment (start 9.15 4.75) (end 9.25 4.65) (width 0.15) (layer "B.Cu") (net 4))
 (segment (start 10.9 8.2) (end 11 8.1) (width 0.15) (layer "B.Cu") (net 4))
 (segment (start 3.35 6.9) (end 3.3 6.95) (width 0.15) (layer "B.Cu") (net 4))
 (segment (start 5.7 2.2) (end 4.3 0.8) (width 0.15) (layer "B.Cu") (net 4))
 (segment (start 7.8 8.5) (end 8.1 8.2) (width 0.15) (layer "B.Cu") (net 4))
 (segment (start 9.25 3.65) (end 7.8 2.2) (width 0.15) (layer "B.Cu") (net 4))
 (segment (start 3.3 9.75) (end 3.35 9.8) (width 0.15) (layer "B.Cu") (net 4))
 (segment (start 7.6 5) (end 7.85 4.75) (width 0.15) (layer "B.Cu") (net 4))
 (segment (start 11 7.1) (end 8.9 5) (width 0.15) (layer "B.Cu") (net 4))
 (segment (start 3.3 6.95) (end 3.3 9.75) (width 0.15) (layer "B.Cu") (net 4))
 (segment (start 8.9 5) (end 7.6 5) (width 0.15) (layer "B.Cu") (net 4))
 (segment (start 9.25 4.65) (end 9.25 3.65) (width 0.15) (layer "B.Cu") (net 4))
 (segment (start 7.6 14.2) (end 6.95 14.85) (width 0.15) (layer "B.Cu") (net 4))
 (segment (start 9.5 10.4) (end 9.5 10.2) (width 0.15) (layer "F.Cu") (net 7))
 (segment (start 9.5 10.2) (end 9.75 9.95) (width 0.15) (layer "F.Cu") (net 7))
 (segment (start 10.3 3.55) (end 9.75 3) (width 0.15) (layer "F.Cu") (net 7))
 (segment (start 8.7 13.8) (end 8.7 11.2) (width 0.15) (layer "F.Cu") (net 7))
 (segment (start 9.75 7) (end 10.3 6.45) (width 0.15) (layer "F.Cu") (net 7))
 (segment (start 8.7 11.2) (end 9.5 10.4) (width 0.15) (layer "F.Cu") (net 7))
 (segment (start 6 14.8) (end 9.5 14.8) (width 0.15) (layer "F.Cu") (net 7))
 (segment (start 5.2 14) (end 6 14.8) (width 0.15) (layer "F.Cu") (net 7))
 (segment (start 10.3 6.45) (end 10.3 3.55) (width 0.15) (layer "F.Cu") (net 7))
 (segment (start 9.75 9.95) (end 9.75 7) (width 0.15) (layer "F.Cu") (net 7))
 (segment (start 9.5 14.6) (end 8.7 13.8) (width 0.15) (layer "F.Cu") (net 7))
 (segment (start 9.75 3) (end 9.75 2.2) (width 0.15) (layer "F.Cu") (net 7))
 (segment (start 9.5 14.8) (end 9.5 14.6) (width 0.15) (layer "F.Cu") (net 7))
 (segment (start 7.55 3.4) (end 6.75 4.2) (width 0.15) (layer "F.Cu") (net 6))
 (segment (start 7.55 2.9) (end 7.55 3.4) (width 0.15) (layer "F.Cu") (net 6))
 (segment (start 5.75 5.95) (end 5.75 6.4) (width 0.15) (layer "F.Cu") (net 6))
 (segment (start 6.75 4.2) (end 6.1 4.2) (width 0.15) (layer "F.Cu") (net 6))
 (segment (start 5.75 7.25) (end 5.75 6.4) (width 0.15) (layer "F.Cu") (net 6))
 (segment (start 6 5.7) (end 5.75 5.95) (width 0.15) (layer "F.Cu") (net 6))
 (segment (start 6 4.3) (end 6 5.7) (width 0.15) (layer "F.Cu") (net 6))
 (segment (start 8.25 2.2) (end 7.55 2.9) (width 0.15) (layer "F.Cu") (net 6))
 (segment (start 6.1 4.2) (end 6 4.3) (width 0.15) (layer "F.Cu") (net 6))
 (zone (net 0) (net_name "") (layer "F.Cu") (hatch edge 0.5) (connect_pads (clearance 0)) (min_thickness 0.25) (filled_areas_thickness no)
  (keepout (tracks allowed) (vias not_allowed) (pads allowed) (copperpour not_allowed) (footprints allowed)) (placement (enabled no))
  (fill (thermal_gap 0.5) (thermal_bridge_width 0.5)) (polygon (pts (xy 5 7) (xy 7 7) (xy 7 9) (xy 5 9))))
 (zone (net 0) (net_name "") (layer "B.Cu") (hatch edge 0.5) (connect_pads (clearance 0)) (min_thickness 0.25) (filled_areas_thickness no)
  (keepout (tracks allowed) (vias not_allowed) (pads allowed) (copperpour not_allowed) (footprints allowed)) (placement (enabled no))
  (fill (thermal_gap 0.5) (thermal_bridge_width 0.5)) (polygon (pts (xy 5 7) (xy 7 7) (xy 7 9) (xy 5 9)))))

